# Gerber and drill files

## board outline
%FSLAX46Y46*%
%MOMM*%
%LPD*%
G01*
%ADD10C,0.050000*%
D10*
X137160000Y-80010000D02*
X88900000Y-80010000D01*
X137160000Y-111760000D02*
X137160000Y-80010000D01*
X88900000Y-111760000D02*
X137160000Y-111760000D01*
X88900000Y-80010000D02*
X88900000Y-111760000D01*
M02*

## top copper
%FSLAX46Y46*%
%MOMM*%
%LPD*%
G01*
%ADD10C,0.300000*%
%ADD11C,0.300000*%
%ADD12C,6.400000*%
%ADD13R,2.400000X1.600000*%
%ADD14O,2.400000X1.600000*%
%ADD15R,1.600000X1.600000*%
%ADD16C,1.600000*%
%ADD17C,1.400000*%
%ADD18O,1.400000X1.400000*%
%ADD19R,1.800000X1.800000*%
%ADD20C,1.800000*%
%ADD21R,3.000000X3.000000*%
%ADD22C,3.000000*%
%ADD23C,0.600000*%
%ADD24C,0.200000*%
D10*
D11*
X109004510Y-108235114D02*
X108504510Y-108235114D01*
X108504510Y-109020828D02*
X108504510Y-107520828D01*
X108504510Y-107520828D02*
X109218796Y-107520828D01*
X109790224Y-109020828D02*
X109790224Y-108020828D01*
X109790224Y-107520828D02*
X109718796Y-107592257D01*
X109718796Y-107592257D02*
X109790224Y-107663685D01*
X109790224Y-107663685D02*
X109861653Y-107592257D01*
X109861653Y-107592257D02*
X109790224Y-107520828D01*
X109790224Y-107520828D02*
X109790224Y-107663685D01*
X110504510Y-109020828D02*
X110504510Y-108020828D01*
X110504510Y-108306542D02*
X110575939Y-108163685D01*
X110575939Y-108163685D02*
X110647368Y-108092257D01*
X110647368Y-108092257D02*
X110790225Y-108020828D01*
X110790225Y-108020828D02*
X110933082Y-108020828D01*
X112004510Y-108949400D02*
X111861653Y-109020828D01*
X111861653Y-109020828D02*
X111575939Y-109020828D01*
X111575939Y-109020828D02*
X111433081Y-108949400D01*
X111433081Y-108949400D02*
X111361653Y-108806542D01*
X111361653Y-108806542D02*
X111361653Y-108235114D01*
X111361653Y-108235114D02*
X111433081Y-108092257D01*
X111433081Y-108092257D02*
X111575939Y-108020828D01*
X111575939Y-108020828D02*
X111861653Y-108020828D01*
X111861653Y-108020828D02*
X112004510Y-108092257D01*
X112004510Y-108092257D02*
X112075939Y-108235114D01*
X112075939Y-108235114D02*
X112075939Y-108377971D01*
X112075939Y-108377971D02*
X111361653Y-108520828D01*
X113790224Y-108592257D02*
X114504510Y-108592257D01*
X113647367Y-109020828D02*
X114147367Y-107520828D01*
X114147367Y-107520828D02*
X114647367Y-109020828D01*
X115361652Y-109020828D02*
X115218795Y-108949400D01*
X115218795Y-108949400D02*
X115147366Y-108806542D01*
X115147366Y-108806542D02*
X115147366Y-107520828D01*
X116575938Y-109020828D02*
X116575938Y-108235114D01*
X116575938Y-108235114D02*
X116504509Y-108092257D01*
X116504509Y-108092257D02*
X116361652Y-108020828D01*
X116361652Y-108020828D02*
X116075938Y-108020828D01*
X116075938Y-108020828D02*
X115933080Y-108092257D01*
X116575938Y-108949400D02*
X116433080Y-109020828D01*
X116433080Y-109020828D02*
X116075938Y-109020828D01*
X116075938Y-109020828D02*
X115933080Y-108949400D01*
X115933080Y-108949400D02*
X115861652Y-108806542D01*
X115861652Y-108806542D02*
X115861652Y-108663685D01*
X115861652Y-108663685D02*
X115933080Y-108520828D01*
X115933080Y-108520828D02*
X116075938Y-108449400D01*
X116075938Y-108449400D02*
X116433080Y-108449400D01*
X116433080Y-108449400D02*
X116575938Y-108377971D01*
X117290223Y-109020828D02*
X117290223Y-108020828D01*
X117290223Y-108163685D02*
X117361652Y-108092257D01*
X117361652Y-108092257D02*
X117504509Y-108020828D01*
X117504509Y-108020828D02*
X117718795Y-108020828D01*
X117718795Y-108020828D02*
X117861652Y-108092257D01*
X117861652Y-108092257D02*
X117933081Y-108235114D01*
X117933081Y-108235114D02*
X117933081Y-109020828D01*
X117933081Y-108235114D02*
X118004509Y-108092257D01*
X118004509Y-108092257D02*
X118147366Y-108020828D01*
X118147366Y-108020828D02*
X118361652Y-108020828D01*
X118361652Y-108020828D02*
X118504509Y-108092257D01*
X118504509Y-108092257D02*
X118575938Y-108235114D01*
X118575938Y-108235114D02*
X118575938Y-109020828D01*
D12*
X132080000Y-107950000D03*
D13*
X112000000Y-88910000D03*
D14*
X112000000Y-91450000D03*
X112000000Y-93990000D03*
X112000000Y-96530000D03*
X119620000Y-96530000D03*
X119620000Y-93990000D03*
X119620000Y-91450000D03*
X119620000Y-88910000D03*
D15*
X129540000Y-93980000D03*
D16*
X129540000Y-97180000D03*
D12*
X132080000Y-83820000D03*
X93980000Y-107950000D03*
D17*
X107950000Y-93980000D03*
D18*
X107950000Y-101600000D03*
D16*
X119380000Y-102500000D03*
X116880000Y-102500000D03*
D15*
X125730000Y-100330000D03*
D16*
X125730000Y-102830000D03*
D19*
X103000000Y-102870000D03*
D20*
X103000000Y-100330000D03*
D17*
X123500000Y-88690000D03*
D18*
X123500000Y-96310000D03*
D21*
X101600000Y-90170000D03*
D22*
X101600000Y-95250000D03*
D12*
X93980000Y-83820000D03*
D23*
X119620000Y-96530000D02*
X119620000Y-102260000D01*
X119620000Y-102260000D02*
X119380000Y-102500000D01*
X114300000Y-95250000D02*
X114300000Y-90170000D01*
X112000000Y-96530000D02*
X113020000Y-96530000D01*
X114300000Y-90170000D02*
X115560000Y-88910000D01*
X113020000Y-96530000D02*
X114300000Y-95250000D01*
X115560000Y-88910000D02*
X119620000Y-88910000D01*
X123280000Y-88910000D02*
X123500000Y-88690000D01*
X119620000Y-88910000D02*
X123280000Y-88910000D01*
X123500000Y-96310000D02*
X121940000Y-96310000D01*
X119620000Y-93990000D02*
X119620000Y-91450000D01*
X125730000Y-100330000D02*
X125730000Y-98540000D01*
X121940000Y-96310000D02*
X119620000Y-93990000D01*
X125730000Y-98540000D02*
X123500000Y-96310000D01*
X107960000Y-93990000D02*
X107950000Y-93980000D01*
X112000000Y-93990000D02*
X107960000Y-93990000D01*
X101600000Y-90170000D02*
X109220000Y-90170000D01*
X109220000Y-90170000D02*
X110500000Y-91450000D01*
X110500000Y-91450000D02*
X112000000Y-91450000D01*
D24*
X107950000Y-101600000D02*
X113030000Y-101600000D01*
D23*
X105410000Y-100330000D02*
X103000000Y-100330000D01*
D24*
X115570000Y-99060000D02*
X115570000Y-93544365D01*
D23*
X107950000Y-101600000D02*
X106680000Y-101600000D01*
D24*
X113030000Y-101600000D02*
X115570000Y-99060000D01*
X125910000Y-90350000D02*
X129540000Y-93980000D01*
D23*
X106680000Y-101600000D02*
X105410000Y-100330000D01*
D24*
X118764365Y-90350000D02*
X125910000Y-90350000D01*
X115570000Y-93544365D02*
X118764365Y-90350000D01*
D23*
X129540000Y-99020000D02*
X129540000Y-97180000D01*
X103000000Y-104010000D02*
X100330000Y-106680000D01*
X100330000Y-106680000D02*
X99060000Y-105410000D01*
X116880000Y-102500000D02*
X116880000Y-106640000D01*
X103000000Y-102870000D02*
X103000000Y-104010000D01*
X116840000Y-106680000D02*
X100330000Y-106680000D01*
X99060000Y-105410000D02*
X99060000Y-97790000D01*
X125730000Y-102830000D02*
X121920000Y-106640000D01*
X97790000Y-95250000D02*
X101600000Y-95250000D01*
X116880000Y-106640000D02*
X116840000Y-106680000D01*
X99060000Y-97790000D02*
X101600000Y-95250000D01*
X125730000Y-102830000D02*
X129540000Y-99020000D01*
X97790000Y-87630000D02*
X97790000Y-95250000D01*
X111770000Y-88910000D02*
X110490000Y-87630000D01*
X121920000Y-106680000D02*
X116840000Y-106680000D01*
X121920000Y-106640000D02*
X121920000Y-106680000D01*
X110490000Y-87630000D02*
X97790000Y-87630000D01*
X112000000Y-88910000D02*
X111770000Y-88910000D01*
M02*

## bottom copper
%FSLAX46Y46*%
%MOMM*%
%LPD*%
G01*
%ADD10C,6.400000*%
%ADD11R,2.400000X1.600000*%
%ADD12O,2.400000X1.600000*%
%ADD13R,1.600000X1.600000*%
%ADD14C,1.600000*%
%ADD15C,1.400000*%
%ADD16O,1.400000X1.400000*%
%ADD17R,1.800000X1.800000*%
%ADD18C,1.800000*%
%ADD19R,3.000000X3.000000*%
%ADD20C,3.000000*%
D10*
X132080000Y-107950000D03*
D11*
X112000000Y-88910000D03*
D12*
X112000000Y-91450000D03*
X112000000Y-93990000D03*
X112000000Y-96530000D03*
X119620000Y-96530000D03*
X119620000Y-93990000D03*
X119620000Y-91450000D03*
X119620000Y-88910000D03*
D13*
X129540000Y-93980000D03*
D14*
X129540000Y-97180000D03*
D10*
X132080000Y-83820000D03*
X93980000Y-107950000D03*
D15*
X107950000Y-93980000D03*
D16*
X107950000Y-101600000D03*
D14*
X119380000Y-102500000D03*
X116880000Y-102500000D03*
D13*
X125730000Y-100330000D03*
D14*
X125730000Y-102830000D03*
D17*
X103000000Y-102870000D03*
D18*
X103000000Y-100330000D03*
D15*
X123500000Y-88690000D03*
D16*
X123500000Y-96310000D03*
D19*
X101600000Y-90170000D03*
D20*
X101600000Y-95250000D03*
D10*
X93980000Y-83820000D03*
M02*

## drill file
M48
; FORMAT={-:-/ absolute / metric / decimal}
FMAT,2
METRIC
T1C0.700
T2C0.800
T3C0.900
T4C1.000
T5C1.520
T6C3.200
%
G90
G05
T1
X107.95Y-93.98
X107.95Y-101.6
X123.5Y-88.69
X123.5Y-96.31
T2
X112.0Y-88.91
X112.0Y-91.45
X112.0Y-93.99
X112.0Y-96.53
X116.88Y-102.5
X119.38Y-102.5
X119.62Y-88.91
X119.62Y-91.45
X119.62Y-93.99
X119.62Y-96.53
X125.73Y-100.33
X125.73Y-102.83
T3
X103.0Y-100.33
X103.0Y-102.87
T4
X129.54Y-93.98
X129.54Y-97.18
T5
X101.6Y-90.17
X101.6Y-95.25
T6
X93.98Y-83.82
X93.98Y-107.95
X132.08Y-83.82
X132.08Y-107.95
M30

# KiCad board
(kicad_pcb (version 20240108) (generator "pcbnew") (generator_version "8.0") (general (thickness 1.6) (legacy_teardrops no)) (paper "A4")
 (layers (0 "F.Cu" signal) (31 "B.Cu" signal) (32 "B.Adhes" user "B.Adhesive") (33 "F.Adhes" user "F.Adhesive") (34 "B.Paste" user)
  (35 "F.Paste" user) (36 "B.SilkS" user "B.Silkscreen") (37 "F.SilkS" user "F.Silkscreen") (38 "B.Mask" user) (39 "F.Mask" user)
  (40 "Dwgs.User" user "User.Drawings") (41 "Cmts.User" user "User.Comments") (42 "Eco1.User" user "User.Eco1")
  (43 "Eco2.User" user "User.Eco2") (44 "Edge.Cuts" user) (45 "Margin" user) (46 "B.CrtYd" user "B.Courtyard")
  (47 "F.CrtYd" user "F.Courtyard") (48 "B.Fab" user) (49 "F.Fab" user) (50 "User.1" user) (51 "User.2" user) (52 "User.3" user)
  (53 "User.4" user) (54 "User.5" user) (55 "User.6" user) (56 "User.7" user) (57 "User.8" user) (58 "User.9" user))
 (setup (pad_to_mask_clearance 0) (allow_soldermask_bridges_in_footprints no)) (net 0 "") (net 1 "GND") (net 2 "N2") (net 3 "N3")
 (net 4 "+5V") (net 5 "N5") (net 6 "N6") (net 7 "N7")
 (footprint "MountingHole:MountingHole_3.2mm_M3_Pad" (layer "F.Cu") (at 132.08 107.95)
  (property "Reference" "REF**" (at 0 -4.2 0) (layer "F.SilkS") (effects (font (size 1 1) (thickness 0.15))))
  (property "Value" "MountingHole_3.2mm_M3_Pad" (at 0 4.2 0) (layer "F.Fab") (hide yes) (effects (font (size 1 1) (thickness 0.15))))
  (pad "1" thru_hole circle (at 0 0) (size 6.4 6.4) (drill 3.2) (layers "*.Cu" "*.Mask") (remove_unused_layers no)))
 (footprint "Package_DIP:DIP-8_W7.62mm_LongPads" (layer "F.Cu") (at 112 88.91)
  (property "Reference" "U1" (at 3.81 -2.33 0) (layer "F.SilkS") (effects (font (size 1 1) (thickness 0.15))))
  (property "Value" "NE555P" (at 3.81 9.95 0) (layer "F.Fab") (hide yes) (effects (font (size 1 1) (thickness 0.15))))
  (pad "1" thru_hole rect (at 0 0) (size 2.4 1.6) (drill 0.8) (layers "*.Cu" "*.Mask") (remove_unused_layers no) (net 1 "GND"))
  (pad "2" thru_hole oval (at 0 2.54) (size 2.4 1.6) (drill 0.8) (layers "*.Cu" "*.Mask") (remove_unused_layers no) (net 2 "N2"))
  (pad "3" thru_hole oval (at 0 5.08) (size 2.4 1.6) (drill 0.8) (layers "*.Cu" "*.Mask") (remove_unused_layers no) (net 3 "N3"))
  (pad "4" thru_hole oval (at 0 7.62) (size 2.4 1.6) (drill 0.8) (layers "*.Cu" "*.Mask") (remove_unused_layers no) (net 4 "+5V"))
  (pad "5" thru_hole oval (at 7.62 7.62) (size 2.4 1.6) (drill 0.8) (layers "*.Cu" "*.Mask") (remove_unused_layers no) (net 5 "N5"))
  (pad "6" thru_hole oval (at 7.62 5.08) (size 2.4 1.6) (drill 0.8) (layers "*.Cu" "*.Mask") (remove_unused_layers no) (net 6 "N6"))
  (pad "7" thru_hole oval (at 7.62 2.54) (size 2.4 1.6) (drill 0.8) (layers "*.Cu" "*.Mask") (remove_unused_layers no) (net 6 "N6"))
  (pad "8" thru_hole oval (at 7.62 0) (size 2.4 1.6) (drill 0.8) (layers "*.Cu" "*.Mask") (remove_unused_layers no) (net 4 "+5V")))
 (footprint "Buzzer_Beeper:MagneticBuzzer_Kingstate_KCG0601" (layer "F.Cu") (at 129.54 93.98 -90)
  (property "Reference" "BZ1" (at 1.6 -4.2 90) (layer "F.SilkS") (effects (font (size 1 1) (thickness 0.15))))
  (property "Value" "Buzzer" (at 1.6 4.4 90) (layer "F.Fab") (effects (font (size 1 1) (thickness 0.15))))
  (pad "1" thru_hole rect (at 0 0 270) (size 1.6 1.6) (drill 1) (layers "*.Cu" "*.Mask") (remove_unused_layers no) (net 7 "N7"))
  (pad "2" thru_hole circle (at 3.2 0 270) (size 1.6 1.6) (drill 1) (layers "*.Cu" "*.Mask") (remove_unused_layers no) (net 1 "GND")))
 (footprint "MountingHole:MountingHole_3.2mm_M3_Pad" (layer "F.Cu") (at 132.08 83.82)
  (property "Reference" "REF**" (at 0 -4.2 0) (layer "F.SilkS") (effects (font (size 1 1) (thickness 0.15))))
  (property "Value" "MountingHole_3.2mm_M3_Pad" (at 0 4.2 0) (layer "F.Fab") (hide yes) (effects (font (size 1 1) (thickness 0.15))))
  (pad "1" thru_hole circle (at 0 0) (size 6.4 6.4) (drill 3.2) (layers "*.Cu" "*.Mask") (remove_unused_layers no)))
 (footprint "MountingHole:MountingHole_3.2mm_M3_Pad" (layer "F.Cu") (at 93.98 107.95)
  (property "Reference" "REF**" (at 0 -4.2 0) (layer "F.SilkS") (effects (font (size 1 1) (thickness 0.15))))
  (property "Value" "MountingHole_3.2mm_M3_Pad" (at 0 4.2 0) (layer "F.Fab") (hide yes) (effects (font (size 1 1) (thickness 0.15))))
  (pad "1" thru_hole circle (at 0 0) (size 6.4 6.4) (drill 3.2) (layers "*.Cu" "*.Mask") (remove_unused_layers no)))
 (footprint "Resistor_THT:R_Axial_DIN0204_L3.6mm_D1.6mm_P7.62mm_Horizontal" (layer "F.Cu") (at 107.95 93.98 -90)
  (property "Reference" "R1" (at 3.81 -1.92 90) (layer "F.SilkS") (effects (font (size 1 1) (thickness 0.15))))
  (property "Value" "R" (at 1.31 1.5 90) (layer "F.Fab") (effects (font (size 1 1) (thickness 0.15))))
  (pad "1" thru_hole circle (at 0 0 270) (size 1.4 1.4) (drill 0.7) (layers "*.Cu" "*.Mask") (remove_unused_layers no) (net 3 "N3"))
  (pad "2" thru_hole oval (at 7.62 0 270) (size 1.4 1.4) (drill 0.7) (layers "*.Cu" "*.Mask") (remove_unused_layers no) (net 7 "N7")))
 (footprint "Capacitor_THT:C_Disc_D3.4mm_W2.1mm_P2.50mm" (layer "F.Cu") (at 119.38 102.5 180)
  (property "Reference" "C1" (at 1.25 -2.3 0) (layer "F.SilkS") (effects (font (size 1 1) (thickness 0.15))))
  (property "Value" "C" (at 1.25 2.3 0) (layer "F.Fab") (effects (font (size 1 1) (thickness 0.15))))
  (pad "1" thru_hole circle (at 0 0 180) (size 1.6 1.6) (drill 0.8) (layers "*.Cu" "*.Mask") (remove_unused_layers no) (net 5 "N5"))
  (pad "2" thru_hole circle (at 2.5 0 180) (size 1.6 1.6) (drill 0.8) (layers "*.Cu" "*.Mask") (remove_unused_layers no) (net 1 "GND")))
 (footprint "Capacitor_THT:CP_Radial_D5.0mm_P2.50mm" (layer "F.Cu") (at 125.73 100.33 -90)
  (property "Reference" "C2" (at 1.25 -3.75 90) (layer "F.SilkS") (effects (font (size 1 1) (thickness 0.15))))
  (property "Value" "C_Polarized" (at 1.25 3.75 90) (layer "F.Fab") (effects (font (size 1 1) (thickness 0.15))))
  (pad "1" thru_hole rect (at 0 0 270) (size 1.6 1.6) (drill 0.8) (layers "*.Cu" "*.Mask") (remove_unused_layers no) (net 6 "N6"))
  (pad "2" thru_hole circle (at 2.5 0 270) (size 1.6 1.6) (drill 0.8) (layers "*.Cu" "*.Mask") (remove_unused_layers no) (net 1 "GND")))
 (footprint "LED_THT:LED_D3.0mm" (layer "F.Cu") (at 103 102.87 90)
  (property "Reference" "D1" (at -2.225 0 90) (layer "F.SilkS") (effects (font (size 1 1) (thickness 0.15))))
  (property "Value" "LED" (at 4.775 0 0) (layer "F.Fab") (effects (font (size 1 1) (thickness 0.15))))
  (pad "1" thru_hole rect (at 0 0 90) (size 1.8 1.8) (drill 0.9) (layers "*.Cu" "*.Mask") (remove_unused_layers no) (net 1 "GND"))
  (pad "2" thru_hole circle (at 2.54 0 90) (size 1.8 1.8) (drill 0.9) (layers "*.Cu" "*.Mask") (remove_unused_layers no) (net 7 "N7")))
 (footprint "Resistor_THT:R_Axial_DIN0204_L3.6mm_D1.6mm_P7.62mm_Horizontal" (layer "F.Cu") (at 123.5 88.69 -90)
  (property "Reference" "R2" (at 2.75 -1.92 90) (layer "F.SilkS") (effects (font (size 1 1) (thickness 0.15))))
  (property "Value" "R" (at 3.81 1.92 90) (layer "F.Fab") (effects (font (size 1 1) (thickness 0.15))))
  (pad "1" thru_hole circle (at 0 0 270) (size 1.4 1.4) (drill 0.7) (layers "*.Cu" "*.Mask") (remove_unused_layers no) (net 4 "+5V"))
  (pad "2" thru_hole oval (at 7.62 0 270) (size 1.4 1.4) (drill 0.7) (layers "*.Cu" "*.Mask") (remove_unused_layers no) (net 6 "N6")))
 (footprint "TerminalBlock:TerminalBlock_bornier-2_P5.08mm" (layer "F.Cu") (at 101.6 90.17 -90)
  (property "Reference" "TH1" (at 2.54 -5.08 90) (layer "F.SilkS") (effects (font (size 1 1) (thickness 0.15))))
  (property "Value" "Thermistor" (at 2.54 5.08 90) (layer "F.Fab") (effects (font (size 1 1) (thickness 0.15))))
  (pad "1" thru_hole rect (at 0 0 270) (size 3 3) (drill 1.52) (layers "*.Cu" "*.Mask") (remove_unused_layers no) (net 2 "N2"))
  (pad "2" thru_hole circle (at 5.08 0 270) (size 3 3) (drill 1.52) (layers "*.Cu" "*.Mask") (remove_unused_layers no) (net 1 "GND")))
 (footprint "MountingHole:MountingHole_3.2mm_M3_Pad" (layer "F.Cu") (at 93.98 83.82)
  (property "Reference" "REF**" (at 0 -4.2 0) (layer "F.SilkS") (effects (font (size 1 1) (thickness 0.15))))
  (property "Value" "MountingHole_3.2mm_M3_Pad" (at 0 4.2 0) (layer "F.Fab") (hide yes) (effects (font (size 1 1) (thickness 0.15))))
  (pad "1" thru_hole circle (at 0 0) (size 6.4 6.4) (drill 3.2) (layers "*.Cu" "*.Mask") (remove_unused_layers no)))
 (gr_line (start 137.16 80.01) (end 88.9 80.01) (stroke (width 0.05) (type default)) (layer "Edge.Cuts"))
 (gr_line (start 137.16 111.76) (end 137.16 80.01) (stroke (width 0.05) (type default)) (layer "Edge.Cuts"))
 (gr_line (start 88.9 111.76) (end 137.16 111.76) (stroke (width 0.05) (type default)) (layer "Edge.Cuts"))
 (gr_line (start 88.9 80.01) (end 88.9 111.76) (stroke (width 0.05) (type default)) (layer "Edge.Cuts"))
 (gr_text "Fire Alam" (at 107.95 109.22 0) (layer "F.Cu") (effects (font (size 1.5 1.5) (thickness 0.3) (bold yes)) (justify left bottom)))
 (segment (start 119.62 96.53) (end 119.62 102.26) (width 0.6) (layer "F.Cu") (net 5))
 (segment (start 119.62 102.26) (end 119.38 102.5) (width 0.6) (layer "F.Cu") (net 5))
 (segment (start 114.3 95.25) (end 114.3 90.17) (width 0.6) (layer "F.Cu") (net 4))
 (segment (start 112 96.53) (end 113.02 96.53) (width 0.6) (layer "F.Cu") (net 4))
 (segment (start 114.3 90.17) (end 115.56 88.91) (width 0.6) (layer "F.Cu") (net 4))
 (segment (start 113.02 96.53) (end 114.3 95.25) (width 0.6) (layer "F.Cu") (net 4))
 (segment (start 115.56 88.91) (end 119.62 88.91) (width 0.6) (layer "F.Cu") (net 4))
 (segment (start 123.28 88.91) (end 123.5 88.69) (width 0.6) (layer "F.Cu") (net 4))
 (segment (start 119.62 88.91) (end 123.28 88.91) (width 0.6) (layer "F.Cu") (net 4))
 (segment (start 123.5 96.31) (end 121.94 96.31) (width 0.6) (layer "F.Cu") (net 6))
 (segment (start 119.62 93.99) (end 119.62 91.45) (width 0.6) (layer "F.Cu") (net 6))
 (segment (start 125.73 100.33) (end 125.73 98.54) (width 0.6) (layer "F.Cu") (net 6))
 (segment (start 121.94 96.31) (end 119.62 93.99) (width 0.6) (layer "F.Cu") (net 6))
 (segment (start 125.73 98.54) (end 123.5 96.31) (width 0.6) (layer "F.Cu") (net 6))
 (segment (start 107.96 93.99) (end 107.95 93.98) (width 0.6) (layer "F.Cu") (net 3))
 (segment (start 112 93.99) (end 107.96 93.99) (width 0.6) (layer "F.Cu") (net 3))
 (segment (start 101.6 90.17) (end 109.22 90.17) (width 0.6) (layer "F.Cu") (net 2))
 (segment (start 109.22 90.17) (end 110.5 91.45) (width 0.6) (layer "F.Cu") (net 2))
 (segment (start 110.5 91.45) (end 112 91.45) (width 0.6) (layer "F.Cu") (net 2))
 (segment (start 107.95 101.6) (end 113.03 101.6) (width 0.2) (layer "F.Cu") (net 7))
 (segment (start 105.41 100.33) (end 103 100.33) (width 0.6) (layer "F.Cu") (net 7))
 (segment (start 115.57 99.06) (end 115.57 93.544365) (width 0.2) (layer "F.Cu") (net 7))
 (segment (start 107.95 101.6) (end 106.68 101.6) (width 0.6) (layer "F.Cu") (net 7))
 (segment (start 113.03 101.6) (end 115.57 99.06) (width 0.2) (layer "F.Cu") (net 7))
 (segment (start 125.91 90.35) (end 129.54 93.98) (width 0.2) (layer "F.Cu") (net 7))
 (segment (start 106.68 101.6) (end 105.41 100.33) (width 0.6) (layer "F.Cu") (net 7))
 (segment (start 118.764365 90.35) (end 125.91 90.35) (width 0.2) (layer "F.Cu") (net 7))
 (segment (start 115.57 93.544365) (end 118.764365 90.35) (width 0.2) (layer "F.Cu") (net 7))
 (segment (start 129.54 99.02) (end 129.54 97.18) (width 0.6) (layer "F.Cu") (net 1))
 (segment (start 103 104.01) (end 100.33 106.68) (width 0.6) (layer "F.Cu") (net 1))
 (segment (start 100.33 106.68) (end 99.06 105.41) (width 0.6) (layer "F.Cu") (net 1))
 (segment (start 116.88 102.5) (end 116.88 106.64) (width 0.6) (layer "F.Cu") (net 1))
 (segment (start 103 102.87) (end 103 104.01) (width 0.6) (layer "F.Cu") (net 1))
 (segment (start 116.84 106.68) (end 100.33 106.68) (width 0.6) (layer "F.Cu") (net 1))
 (segment (start 99.06 105.41) (end 99.06 97.79) (width 0.6) (layer "F.Cu") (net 1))
 (segment (start 125.73 102.83) (end 121.92 106.64) (width 0.6) (layer "F.Cu") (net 1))
 (segment (start 97.79 95.25) (end 101.6 95.25) (width 0.6) (layer "F.Cu") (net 1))
 (segment (start 116.88 106.64) (end 116.84 106.68) (width 0.6) (layer "F.Cu") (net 1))
 (segment (start 99.06 97.79) (end 101.6 95.25) (width 0.6) (layer "F.Cu") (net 1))
 (segment (start 125.73 102.83) (end 129.54 99.02) (width 0.6) (layer "F.Cu") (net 1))
 (segment (start 97.79 87.63) (end 97.79 95.25) (width 0.6) (layer "F.Cu") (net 1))
 (segment (start 111.77 88.91) (end 110.49 87.63) (width 0.6) (layer "F.Cu") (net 1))
 (segment (start 121.92 106.68) (end 116.84 106.68) (width 0.6) (layer "F.Cu") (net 1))
 (segment (start 121.92 106.64) (end 121.92 106.68) (width 0.6) (layer "F.Cu") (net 1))
 (segment (start 110.49 87.63) (end 97.79 87.63) (width 0.6) (layer "F.Cu") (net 1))
 (segment (start 112 88.91) (end 111.77 88.91) (width 0.6) (layer "F.Cu") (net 1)))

